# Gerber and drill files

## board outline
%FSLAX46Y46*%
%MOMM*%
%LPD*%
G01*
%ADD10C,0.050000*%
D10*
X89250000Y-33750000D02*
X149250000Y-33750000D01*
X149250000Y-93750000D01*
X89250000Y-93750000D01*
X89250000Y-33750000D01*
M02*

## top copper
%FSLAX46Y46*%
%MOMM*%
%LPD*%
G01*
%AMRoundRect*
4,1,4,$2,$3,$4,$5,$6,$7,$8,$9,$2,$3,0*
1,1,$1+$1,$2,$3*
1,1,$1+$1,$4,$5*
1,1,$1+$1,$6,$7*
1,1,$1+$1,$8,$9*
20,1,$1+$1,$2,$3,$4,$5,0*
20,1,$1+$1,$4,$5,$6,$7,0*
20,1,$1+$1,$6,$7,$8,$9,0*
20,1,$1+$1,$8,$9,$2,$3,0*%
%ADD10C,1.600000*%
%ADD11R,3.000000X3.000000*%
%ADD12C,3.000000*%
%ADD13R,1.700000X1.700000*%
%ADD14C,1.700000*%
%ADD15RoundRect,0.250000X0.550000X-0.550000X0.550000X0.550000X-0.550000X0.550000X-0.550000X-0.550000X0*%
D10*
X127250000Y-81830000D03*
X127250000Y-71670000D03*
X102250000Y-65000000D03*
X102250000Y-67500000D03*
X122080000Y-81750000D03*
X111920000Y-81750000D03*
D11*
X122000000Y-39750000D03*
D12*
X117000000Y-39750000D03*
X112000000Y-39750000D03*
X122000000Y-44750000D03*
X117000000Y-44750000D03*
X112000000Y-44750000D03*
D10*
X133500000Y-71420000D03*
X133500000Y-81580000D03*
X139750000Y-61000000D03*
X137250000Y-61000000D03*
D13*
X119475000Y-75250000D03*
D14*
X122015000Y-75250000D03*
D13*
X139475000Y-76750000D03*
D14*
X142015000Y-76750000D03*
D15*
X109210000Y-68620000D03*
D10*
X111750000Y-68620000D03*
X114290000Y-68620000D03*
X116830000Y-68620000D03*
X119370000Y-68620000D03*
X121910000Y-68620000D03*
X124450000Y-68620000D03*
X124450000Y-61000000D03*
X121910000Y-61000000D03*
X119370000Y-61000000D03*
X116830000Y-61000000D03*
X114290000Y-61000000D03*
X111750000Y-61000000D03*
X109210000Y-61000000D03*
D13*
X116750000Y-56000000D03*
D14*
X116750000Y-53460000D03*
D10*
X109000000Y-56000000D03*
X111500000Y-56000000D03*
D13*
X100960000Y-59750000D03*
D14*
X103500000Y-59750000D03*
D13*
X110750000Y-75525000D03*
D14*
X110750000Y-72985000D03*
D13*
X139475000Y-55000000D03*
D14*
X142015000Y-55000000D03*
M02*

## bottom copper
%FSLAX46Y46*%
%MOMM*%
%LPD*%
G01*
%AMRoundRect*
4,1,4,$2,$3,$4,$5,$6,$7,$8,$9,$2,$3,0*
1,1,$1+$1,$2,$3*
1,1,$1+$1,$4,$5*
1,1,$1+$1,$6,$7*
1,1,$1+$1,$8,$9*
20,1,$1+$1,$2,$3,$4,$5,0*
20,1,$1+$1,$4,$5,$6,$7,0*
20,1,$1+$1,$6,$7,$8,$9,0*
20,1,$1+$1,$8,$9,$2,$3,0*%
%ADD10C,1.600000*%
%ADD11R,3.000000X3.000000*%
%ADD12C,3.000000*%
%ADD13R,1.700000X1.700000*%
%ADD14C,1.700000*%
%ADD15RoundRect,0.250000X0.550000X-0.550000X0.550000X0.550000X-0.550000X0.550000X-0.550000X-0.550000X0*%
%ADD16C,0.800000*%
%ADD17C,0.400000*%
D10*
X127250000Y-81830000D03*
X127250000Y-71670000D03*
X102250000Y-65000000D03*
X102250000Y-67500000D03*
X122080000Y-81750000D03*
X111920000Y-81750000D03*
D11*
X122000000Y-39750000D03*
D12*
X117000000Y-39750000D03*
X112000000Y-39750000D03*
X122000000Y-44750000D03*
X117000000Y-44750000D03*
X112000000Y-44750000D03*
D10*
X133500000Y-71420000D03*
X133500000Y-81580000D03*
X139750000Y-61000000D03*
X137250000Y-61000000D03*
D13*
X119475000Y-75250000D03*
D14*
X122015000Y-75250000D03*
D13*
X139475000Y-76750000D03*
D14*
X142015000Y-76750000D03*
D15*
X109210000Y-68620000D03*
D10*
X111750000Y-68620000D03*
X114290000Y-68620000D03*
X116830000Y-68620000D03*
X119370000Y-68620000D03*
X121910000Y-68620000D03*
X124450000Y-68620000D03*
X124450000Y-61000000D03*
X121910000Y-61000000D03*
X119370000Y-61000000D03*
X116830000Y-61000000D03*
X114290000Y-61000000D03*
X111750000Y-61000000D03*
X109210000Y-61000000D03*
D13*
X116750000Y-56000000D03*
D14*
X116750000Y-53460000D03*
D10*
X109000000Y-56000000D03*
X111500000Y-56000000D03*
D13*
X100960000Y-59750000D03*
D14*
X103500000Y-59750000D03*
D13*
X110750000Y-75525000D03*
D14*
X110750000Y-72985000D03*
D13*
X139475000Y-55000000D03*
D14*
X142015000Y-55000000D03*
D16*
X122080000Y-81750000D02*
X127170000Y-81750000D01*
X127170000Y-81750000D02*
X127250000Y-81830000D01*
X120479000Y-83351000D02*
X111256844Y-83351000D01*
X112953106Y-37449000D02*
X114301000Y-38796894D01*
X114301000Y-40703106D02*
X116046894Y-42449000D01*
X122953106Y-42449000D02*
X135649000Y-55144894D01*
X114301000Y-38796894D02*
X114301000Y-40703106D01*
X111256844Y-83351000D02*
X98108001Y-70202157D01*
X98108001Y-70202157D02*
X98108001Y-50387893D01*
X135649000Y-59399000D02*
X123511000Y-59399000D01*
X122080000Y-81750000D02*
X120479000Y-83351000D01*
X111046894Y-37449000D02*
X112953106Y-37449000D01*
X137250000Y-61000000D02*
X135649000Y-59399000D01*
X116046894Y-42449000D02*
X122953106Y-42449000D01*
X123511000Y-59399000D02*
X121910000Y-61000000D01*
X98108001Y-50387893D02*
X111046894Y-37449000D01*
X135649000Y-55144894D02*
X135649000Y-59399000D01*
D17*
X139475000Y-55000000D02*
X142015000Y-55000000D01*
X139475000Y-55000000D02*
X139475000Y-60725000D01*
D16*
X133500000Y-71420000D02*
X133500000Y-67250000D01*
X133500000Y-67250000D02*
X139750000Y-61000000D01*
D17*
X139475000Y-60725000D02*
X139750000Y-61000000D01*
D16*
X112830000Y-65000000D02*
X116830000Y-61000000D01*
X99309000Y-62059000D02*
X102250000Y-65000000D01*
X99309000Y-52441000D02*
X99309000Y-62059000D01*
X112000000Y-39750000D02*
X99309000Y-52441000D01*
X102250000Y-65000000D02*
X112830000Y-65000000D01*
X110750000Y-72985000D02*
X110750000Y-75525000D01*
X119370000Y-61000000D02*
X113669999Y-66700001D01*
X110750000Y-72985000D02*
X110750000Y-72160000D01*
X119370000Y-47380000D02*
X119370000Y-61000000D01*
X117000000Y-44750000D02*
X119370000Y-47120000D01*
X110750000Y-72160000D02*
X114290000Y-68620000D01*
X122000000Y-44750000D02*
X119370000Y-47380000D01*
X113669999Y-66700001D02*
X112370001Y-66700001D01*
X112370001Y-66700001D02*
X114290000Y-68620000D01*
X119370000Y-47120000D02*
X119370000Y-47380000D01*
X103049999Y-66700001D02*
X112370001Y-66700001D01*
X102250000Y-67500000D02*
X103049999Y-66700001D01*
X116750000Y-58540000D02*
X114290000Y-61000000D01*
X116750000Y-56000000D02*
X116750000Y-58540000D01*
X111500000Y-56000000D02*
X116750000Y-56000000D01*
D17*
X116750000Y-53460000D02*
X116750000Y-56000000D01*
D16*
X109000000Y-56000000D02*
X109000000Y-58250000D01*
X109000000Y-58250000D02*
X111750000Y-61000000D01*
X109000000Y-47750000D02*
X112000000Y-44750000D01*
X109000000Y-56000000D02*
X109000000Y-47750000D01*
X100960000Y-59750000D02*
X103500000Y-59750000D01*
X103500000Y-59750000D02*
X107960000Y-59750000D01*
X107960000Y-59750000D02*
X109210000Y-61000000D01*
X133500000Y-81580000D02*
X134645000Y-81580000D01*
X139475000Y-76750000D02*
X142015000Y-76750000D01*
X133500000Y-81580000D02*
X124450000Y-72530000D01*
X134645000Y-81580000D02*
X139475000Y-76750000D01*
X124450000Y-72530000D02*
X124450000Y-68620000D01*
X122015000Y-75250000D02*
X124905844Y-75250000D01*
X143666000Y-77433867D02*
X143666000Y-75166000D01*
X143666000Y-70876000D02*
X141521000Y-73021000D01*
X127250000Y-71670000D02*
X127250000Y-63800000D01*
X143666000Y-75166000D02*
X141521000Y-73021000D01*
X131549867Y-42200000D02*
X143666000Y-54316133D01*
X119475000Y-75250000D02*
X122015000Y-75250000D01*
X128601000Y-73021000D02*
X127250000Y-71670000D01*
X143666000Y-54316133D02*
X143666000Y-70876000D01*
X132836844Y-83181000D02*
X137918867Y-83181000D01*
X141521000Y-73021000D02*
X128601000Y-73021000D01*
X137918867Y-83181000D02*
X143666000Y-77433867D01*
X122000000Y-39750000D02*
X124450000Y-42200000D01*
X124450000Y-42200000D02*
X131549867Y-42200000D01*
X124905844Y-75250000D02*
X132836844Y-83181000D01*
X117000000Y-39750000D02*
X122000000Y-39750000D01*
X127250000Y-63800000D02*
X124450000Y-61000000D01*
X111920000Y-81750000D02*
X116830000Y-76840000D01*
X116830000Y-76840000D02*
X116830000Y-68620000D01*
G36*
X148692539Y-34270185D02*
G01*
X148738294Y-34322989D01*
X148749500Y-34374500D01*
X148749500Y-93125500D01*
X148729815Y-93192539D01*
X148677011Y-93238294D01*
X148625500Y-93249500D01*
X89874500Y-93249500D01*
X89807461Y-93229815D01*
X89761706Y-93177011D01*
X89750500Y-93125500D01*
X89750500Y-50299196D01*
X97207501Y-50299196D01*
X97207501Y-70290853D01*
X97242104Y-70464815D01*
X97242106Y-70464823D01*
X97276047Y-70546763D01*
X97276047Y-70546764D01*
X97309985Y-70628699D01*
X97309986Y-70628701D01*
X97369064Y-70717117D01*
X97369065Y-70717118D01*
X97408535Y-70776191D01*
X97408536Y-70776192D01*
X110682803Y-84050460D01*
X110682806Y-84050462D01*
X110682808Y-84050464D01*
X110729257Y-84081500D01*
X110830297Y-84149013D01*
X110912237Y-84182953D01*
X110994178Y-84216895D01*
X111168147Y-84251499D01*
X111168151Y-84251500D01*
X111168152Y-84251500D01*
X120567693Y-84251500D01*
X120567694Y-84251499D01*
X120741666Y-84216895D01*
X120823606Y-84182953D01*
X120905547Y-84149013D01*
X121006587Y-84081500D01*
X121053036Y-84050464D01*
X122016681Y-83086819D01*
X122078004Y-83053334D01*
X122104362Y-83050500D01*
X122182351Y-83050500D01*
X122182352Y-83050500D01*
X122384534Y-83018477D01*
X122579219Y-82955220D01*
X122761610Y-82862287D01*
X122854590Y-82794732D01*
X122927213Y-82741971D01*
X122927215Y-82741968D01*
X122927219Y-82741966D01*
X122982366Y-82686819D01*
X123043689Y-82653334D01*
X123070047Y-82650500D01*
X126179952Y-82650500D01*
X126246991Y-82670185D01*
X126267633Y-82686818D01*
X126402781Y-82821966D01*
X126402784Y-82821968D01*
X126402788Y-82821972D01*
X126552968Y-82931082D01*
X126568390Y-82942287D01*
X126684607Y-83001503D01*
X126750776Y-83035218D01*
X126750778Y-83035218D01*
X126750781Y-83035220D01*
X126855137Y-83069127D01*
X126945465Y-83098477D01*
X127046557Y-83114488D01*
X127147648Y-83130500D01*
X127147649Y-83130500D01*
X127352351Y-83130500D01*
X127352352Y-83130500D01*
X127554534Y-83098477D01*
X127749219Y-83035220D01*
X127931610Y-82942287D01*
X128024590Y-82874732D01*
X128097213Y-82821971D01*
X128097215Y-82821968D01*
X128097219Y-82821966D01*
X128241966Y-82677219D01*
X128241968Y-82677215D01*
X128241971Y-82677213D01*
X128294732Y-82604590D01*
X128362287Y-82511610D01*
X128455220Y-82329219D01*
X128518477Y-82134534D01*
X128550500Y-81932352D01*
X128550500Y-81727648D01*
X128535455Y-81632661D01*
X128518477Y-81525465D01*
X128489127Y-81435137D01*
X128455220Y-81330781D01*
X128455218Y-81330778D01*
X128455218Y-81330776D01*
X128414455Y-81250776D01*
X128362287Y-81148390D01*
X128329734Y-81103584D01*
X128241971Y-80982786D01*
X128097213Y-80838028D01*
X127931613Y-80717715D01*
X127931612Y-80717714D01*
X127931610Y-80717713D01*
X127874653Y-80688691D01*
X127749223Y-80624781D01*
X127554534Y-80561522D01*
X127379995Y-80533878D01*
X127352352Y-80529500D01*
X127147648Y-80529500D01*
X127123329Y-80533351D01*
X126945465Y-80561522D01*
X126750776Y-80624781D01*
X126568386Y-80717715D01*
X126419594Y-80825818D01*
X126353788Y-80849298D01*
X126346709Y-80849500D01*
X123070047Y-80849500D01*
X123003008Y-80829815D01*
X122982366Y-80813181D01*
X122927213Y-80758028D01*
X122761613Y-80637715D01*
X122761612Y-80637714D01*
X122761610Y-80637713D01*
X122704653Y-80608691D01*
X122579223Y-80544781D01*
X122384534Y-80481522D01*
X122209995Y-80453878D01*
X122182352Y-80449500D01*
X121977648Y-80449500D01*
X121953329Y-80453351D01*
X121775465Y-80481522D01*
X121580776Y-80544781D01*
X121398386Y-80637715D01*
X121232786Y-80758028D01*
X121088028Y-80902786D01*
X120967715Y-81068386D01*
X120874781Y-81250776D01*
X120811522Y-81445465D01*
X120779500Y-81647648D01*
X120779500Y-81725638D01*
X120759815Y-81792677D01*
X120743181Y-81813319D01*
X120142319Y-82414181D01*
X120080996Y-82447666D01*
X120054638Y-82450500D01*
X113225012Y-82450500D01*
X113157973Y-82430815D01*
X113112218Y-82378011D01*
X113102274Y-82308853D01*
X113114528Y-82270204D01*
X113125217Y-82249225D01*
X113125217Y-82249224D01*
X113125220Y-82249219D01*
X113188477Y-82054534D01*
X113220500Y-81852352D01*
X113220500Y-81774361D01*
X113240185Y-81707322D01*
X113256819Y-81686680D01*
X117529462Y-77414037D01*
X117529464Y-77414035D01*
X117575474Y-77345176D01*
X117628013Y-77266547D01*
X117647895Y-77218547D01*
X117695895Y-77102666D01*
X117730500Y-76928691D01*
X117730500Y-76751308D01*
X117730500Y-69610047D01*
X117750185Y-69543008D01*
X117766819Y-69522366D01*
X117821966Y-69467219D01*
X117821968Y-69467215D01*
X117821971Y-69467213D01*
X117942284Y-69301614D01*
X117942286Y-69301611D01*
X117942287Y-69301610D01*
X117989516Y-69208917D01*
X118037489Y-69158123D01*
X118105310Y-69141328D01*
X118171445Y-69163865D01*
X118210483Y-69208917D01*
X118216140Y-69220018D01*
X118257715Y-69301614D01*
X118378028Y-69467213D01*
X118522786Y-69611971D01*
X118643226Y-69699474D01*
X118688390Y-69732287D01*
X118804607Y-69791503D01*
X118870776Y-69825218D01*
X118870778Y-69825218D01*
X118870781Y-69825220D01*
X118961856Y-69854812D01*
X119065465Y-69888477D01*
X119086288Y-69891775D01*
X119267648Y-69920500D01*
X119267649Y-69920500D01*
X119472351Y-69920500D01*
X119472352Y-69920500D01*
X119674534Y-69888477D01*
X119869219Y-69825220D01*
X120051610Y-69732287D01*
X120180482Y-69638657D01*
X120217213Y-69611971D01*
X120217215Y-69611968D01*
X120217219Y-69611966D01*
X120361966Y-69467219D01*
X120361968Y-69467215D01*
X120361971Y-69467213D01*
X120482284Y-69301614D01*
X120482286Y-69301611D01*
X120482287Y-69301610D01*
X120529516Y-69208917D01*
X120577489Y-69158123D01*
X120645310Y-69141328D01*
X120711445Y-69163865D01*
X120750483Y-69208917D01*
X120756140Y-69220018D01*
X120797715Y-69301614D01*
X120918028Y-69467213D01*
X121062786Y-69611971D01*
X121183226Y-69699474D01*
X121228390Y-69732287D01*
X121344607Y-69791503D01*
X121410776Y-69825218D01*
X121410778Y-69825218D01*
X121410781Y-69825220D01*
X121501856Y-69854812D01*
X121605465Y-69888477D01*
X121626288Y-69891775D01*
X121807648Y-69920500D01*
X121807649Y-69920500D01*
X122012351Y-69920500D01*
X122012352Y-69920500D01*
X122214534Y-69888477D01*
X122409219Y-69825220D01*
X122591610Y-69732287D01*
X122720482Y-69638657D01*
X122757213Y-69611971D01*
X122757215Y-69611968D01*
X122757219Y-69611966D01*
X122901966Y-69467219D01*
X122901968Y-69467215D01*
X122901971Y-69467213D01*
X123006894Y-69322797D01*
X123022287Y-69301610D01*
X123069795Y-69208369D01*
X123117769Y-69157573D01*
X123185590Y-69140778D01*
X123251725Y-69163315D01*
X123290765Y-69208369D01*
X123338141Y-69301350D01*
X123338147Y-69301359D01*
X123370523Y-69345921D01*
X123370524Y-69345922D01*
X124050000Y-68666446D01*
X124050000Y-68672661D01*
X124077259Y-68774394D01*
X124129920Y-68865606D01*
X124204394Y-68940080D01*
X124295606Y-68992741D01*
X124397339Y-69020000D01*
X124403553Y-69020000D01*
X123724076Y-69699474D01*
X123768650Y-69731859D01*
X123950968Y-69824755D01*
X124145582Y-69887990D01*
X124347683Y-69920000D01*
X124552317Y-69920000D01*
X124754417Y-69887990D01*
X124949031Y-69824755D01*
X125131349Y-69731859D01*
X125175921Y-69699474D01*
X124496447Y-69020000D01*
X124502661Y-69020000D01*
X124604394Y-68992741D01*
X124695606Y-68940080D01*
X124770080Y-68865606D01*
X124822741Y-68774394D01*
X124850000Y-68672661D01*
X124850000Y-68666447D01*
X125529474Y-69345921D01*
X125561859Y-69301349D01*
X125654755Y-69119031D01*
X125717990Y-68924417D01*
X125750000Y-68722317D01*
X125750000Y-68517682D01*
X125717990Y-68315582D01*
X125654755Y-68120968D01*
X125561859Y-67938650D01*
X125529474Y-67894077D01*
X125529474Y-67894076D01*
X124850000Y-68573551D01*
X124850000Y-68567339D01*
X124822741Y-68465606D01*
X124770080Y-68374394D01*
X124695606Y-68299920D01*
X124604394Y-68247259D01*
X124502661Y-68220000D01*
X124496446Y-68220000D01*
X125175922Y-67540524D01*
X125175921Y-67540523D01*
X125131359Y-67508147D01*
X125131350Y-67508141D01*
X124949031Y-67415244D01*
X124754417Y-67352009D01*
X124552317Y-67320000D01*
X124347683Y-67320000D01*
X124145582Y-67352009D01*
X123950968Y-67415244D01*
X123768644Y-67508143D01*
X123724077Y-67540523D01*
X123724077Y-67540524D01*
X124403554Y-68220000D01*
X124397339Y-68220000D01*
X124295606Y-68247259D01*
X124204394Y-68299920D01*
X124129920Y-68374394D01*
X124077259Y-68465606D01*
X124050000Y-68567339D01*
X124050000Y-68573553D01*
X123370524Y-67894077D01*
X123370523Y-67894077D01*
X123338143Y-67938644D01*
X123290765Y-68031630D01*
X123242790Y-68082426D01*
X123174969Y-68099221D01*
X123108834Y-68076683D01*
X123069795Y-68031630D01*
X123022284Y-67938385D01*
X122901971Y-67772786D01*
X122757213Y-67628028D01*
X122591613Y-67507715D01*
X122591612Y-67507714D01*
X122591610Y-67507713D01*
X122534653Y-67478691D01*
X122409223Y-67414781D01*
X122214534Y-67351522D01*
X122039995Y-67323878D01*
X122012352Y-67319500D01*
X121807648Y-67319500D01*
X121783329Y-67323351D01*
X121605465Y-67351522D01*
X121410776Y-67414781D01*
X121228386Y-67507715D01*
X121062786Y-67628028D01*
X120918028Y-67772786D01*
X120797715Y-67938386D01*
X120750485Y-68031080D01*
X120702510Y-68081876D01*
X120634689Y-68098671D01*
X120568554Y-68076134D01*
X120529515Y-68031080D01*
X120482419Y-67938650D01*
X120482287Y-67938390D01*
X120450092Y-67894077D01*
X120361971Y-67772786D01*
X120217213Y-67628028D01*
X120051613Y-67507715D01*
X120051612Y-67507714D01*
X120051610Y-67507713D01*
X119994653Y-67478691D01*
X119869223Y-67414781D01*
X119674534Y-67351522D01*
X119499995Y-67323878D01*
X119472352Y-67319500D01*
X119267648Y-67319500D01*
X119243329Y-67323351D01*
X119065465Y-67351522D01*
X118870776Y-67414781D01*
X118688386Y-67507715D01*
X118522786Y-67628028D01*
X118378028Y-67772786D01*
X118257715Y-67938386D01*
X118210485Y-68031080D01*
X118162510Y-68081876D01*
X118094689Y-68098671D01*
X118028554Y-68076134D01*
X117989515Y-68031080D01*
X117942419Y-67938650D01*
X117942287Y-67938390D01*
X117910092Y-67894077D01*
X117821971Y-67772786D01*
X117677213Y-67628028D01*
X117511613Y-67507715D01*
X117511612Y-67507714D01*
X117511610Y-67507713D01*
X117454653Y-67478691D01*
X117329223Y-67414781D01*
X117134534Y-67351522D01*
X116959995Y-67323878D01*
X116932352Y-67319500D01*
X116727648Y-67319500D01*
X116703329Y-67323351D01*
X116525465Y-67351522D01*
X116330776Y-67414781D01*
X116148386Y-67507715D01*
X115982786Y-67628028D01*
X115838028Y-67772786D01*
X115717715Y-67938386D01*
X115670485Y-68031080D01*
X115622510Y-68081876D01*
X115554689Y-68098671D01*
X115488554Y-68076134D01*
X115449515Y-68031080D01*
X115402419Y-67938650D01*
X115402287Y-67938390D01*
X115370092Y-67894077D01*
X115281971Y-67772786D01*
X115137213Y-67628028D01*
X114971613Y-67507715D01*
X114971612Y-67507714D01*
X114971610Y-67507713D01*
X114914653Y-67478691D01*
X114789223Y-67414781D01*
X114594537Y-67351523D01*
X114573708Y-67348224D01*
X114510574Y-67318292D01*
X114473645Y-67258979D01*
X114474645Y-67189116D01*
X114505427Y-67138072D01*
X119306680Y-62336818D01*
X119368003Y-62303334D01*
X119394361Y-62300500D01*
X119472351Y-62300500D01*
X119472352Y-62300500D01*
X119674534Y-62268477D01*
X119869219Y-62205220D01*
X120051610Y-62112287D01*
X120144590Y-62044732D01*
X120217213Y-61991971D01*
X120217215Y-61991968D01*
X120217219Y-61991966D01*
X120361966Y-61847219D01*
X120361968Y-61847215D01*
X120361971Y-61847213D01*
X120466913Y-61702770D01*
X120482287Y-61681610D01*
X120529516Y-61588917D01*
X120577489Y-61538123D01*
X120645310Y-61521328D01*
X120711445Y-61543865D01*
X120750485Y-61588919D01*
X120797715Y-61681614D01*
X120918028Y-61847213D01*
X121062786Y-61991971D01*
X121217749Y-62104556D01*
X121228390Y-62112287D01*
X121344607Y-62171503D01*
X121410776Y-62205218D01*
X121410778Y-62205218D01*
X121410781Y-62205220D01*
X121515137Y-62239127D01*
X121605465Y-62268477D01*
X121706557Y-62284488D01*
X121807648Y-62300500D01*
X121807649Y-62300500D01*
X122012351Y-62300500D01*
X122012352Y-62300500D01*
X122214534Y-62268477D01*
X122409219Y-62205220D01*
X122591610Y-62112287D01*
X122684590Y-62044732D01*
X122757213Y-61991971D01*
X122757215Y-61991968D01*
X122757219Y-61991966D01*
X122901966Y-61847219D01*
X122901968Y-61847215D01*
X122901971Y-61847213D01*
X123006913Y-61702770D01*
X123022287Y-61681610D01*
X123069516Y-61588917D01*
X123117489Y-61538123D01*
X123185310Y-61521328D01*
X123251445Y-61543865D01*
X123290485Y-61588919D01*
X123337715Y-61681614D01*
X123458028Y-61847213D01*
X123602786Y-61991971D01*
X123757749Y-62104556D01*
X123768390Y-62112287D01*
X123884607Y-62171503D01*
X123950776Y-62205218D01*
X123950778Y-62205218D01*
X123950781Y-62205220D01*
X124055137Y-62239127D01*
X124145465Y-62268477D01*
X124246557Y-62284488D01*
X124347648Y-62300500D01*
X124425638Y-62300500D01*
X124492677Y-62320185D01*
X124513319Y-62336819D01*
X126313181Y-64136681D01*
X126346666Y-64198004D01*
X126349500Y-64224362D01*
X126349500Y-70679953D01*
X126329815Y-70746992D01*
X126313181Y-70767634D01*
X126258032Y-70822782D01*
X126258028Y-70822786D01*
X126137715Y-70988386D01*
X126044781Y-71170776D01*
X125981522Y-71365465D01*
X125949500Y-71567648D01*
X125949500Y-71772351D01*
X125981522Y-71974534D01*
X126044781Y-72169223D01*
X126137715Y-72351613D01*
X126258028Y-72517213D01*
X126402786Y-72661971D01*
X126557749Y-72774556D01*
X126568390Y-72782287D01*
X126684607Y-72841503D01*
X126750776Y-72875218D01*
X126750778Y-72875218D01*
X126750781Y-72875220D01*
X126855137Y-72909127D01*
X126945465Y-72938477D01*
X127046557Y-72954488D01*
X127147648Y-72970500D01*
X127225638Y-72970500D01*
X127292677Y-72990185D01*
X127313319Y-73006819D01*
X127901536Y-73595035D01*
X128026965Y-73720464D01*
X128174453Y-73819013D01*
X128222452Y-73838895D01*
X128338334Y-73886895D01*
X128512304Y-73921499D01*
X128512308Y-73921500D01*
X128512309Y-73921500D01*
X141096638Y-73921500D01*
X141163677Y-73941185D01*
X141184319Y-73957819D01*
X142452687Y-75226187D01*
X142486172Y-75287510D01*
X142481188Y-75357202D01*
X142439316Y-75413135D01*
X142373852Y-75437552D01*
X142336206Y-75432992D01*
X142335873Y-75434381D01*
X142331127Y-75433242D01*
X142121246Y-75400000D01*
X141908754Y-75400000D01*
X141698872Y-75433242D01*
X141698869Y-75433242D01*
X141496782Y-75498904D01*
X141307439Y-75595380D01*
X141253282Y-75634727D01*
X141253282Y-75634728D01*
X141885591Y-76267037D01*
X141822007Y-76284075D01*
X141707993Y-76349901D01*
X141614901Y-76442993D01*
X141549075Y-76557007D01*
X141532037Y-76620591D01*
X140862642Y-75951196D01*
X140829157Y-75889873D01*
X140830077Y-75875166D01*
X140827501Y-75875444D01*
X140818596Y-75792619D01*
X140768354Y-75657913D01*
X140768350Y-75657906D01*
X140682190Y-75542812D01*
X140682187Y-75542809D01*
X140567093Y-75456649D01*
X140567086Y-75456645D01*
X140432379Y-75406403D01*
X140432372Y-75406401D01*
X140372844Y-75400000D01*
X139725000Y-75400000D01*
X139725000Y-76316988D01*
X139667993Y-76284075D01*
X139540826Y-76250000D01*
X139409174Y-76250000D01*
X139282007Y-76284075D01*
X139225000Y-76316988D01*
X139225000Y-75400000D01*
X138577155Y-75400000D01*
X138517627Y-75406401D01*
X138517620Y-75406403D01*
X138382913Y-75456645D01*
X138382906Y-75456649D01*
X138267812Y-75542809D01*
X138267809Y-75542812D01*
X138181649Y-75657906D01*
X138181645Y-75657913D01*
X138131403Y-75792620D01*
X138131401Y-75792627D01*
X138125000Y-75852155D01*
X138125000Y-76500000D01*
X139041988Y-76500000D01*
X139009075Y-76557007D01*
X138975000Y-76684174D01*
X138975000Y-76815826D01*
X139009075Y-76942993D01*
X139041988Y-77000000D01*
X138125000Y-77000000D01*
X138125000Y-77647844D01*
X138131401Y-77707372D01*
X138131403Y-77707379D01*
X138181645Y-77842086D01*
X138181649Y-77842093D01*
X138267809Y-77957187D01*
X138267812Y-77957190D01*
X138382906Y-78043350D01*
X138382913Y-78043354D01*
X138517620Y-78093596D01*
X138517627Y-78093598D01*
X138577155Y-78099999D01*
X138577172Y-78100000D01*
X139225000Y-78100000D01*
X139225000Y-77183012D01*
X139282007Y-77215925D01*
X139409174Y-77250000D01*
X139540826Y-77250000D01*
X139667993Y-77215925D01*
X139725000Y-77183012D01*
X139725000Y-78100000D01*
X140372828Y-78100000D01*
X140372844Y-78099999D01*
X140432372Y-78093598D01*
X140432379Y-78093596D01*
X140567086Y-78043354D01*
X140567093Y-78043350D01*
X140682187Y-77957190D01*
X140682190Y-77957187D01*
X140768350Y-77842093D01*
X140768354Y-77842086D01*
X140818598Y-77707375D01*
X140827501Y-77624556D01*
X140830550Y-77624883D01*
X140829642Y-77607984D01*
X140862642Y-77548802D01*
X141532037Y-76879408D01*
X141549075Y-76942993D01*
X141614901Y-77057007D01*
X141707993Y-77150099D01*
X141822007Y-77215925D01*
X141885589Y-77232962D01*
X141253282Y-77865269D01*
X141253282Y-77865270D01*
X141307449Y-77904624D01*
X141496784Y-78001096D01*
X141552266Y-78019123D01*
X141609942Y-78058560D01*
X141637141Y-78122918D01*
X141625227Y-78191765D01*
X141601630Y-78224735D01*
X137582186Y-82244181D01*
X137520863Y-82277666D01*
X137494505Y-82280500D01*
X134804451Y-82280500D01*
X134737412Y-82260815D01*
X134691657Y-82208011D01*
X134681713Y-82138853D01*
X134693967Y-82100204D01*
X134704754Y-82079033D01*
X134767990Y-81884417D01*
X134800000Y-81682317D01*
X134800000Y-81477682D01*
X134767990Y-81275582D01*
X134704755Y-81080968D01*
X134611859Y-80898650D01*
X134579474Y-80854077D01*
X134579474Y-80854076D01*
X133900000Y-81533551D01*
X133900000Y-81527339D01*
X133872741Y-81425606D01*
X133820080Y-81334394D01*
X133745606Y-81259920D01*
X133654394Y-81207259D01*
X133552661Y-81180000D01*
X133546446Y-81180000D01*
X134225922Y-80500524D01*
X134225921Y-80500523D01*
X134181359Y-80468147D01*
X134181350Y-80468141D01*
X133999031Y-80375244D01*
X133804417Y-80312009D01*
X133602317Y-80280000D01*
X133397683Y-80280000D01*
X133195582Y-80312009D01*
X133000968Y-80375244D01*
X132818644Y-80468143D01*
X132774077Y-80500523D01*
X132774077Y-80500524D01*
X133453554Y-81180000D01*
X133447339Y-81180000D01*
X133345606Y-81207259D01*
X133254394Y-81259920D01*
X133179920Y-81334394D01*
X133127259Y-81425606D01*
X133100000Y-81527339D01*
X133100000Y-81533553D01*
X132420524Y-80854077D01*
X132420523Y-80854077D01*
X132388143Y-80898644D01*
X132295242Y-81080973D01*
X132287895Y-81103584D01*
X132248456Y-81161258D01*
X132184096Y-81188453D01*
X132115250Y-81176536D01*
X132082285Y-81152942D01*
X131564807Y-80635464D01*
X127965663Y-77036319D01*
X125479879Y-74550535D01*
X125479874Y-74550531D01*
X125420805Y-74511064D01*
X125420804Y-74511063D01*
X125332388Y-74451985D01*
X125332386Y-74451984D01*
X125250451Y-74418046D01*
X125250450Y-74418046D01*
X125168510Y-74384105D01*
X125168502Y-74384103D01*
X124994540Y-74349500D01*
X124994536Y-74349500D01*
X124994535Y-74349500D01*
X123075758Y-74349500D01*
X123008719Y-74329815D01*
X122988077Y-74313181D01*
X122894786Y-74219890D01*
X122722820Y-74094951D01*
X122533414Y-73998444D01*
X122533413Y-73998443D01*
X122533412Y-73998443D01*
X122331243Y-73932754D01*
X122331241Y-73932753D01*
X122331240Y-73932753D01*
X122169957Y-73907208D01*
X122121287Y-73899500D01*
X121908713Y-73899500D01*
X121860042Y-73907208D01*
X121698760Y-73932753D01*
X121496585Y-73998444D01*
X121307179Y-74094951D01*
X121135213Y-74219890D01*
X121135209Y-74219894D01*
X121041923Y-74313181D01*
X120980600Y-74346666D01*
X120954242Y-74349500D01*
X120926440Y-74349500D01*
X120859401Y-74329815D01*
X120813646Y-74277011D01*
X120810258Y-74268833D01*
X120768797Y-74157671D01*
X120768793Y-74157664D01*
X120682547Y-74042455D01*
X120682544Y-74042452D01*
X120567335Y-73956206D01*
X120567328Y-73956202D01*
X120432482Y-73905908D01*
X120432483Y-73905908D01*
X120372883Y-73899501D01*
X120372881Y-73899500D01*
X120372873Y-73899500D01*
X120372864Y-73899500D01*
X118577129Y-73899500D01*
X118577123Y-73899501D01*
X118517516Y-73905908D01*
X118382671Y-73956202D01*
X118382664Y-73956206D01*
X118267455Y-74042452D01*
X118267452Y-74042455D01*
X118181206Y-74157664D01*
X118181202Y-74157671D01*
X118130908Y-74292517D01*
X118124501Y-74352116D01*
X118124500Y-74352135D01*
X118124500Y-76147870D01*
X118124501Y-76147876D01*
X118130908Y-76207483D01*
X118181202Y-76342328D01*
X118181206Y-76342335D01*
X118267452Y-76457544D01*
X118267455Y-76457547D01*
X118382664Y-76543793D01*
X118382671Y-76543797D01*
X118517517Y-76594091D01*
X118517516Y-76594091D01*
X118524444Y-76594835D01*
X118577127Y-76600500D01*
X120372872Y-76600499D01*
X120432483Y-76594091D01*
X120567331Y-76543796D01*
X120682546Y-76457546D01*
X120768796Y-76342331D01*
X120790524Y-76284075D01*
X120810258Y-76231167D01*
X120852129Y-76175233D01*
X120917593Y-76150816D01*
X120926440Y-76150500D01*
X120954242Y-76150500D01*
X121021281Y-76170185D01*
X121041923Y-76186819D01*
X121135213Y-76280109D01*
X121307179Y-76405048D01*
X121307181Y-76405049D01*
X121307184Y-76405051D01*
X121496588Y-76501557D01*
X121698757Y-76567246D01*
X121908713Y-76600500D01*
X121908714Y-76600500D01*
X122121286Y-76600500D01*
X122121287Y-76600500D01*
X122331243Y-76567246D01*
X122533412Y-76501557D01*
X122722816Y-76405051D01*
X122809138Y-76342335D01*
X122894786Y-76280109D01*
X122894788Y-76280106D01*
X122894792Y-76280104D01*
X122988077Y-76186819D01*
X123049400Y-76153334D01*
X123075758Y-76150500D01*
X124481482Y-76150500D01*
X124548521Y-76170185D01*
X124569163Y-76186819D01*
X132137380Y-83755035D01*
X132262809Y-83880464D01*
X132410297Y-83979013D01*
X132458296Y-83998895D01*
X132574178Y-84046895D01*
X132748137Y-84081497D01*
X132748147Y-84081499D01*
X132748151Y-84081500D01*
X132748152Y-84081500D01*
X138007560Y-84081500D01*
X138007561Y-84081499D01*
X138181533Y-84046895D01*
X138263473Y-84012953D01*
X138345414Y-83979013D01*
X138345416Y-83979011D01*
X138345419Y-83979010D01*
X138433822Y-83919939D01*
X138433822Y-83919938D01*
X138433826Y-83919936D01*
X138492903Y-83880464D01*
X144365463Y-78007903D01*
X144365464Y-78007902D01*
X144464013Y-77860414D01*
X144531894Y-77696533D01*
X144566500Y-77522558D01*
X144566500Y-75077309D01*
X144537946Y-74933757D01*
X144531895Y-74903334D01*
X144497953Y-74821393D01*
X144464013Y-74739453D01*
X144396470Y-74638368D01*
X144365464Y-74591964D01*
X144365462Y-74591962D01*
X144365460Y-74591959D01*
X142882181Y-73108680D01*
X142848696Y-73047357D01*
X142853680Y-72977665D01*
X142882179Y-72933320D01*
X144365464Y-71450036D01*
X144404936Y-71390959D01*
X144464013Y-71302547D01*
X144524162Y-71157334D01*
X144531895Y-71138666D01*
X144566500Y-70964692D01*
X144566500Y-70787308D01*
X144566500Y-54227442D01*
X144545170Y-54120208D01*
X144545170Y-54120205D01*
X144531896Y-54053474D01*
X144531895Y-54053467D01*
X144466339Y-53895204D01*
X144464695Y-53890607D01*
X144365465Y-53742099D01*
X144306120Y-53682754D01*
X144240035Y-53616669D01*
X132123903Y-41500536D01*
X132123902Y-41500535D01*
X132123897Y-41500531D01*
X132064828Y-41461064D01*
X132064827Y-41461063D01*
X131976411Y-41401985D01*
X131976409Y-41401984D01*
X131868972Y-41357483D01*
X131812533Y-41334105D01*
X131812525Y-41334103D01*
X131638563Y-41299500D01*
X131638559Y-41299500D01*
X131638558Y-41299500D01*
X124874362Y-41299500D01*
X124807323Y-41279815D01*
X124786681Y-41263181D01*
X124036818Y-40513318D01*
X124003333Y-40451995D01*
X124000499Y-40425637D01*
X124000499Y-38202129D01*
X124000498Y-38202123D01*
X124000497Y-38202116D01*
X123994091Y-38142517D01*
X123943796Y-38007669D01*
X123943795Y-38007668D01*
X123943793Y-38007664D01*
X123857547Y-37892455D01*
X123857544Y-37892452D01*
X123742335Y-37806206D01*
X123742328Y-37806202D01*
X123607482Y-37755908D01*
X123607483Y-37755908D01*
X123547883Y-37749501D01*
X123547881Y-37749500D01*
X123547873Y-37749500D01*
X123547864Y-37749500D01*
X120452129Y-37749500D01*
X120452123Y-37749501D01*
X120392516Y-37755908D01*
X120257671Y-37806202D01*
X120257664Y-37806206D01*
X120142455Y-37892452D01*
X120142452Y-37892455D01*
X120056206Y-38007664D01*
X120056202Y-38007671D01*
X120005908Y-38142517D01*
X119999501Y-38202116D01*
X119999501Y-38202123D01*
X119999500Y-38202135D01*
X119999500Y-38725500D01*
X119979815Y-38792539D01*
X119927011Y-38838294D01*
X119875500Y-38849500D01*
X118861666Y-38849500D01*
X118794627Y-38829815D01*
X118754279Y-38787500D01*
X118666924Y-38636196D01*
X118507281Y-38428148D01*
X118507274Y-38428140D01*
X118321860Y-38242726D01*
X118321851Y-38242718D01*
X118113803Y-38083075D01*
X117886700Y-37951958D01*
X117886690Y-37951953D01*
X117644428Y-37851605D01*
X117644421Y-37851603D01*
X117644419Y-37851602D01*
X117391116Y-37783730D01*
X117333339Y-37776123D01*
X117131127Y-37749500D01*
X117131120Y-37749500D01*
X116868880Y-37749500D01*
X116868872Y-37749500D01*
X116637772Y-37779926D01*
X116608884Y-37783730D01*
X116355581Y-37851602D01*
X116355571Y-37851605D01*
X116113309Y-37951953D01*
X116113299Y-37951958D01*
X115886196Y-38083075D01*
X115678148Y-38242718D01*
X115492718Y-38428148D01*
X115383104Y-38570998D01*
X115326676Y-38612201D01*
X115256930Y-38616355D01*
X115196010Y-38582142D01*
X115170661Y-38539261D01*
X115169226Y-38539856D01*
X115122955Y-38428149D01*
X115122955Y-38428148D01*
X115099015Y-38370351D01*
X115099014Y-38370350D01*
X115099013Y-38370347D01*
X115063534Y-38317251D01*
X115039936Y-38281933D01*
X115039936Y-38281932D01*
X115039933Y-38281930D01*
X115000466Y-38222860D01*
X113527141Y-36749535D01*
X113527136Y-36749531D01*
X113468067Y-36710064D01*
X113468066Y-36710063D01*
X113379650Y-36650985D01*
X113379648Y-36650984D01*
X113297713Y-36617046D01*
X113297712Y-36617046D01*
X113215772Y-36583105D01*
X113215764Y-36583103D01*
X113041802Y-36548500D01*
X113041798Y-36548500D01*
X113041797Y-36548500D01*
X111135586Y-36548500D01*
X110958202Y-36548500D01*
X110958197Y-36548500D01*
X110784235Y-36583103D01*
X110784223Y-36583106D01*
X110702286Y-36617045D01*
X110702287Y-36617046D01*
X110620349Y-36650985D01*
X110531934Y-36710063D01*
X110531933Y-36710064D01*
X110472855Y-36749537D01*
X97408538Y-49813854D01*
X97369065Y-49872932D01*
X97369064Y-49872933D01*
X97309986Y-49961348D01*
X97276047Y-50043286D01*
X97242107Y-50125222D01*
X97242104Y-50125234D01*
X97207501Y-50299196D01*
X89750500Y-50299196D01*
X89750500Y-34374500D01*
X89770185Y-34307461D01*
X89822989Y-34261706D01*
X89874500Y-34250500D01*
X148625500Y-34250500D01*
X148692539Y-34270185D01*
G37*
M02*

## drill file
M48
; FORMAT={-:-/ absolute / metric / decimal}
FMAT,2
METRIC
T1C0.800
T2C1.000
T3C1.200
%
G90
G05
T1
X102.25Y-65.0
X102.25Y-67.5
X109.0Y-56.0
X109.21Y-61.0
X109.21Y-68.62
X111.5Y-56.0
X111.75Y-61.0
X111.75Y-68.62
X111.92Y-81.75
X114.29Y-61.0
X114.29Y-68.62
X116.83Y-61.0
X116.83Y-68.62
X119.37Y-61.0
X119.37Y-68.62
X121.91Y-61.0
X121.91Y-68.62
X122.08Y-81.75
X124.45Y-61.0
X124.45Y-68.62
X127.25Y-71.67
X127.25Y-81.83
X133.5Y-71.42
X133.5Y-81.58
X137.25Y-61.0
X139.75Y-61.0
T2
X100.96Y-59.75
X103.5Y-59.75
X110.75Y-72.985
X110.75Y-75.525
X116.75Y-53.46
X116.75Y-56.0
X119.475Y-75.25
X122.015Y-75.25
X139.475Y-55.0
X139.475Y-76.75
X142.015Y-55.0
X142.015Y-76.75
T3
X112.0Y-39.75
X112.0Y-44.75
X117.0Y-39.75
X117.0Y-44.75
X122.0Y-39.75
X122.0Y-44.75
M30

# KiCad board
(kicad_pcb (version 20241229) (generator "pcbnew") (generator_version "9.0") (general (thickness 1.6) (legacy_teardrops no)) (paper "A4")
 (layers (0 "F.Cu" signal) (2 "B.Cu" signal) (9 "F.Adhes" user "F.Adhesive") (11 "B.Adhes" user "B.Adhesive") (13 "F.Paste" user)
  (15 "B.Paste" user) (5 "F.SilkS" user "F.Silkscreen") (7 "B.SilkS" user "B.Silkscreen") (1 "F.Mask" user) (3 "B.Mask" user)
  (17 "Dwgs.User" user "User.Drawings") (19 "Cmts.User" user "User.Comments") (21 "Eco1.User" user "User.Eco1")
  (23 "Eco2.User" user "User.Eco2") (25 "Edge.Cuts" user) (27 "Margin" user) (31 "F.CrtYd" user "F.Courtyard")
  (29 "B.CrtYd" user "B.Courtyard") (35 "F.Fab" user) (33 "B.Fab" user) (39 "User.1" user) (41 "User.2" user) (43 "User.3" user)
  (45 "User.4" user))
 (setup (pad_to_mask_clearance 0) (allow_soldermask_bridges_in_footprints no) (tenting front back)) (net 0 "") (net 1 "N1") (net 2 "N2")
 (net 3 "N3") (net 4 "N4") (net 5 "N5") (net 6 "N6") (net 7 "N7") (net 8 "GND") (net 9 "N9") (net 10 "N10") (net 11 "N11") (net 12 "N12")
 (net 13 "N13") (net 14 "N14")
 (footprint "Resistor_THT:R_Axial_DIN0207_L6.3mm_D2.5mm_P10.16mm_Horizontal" (layer "F.Cu") (at 127.25 81.83 90)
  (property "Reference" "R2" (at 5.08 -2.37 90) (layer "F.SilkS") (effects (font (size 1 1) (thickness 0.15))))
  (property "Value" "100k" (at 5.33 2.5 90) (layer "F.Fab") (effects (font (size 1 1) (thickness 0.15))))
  (pad "1" thru_hole circle (at 0 0 90) (size 1.6 1.6) (drill 0.8) (layers "*.Cu" "*.Mask") (remove_unused_layers no) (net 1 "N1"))
  (pad "2" thru_hole circle (at 10.16 0 90) (size 1.6 1.6) (drill 0.8) (layers "*.Cu" "*.Mask") (remove_unused_layers no) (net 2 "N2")))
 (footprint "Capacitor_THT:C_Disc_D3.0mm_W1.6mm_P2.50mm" (layer "F.Cu") (at 102.25 65 -90)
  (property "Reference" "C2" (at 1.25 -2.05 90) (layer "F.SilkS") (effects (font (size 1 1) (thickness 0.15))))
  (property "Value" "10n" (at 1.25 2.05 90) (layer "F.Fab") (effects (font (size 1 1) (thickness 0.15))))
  (pad "1" thru_hole circle (at 0 0 270) (size 1.6 1.6) (drill 0.8) (layers "*.Cu" "*.Mask") (remove_unused_layers no) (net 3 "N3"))
  (pad "2" thru_hole circle (at 2.5 0 270) (size 1.6 1.6) (drill 0.8) (layers "*.Cu" "*.Mask") (remove_unused_layers no) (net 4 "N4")))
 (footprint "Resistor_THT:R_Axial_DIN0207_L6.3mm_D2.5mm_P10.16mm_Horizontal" (layer "F.Cu") (at 122.08 81.75 180)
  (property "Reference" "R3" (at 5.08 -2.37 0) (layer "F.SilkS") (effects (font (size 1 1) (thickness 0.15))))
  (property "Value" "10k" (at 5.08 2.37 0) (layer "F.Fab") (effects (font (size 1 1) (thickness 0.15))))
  (pad "1" thru_hole circle (at 0 0 180) (size 1.6 1.6) (drill 0.8) (layers "*.Cu" "*.Mask") (remove_unused_layers no) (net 1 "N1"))
  (pad "2" thru_hole circle (at 10.16 0 180) (size 1.6 1.6) (drill 0.8) (layers "*.Cu" "*.Mask") (remove_unused_layers no) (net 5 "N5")))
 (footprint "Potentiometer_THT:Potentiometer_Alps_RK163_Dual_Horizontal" (layer "F.Cu") (at 122 39.75 -90)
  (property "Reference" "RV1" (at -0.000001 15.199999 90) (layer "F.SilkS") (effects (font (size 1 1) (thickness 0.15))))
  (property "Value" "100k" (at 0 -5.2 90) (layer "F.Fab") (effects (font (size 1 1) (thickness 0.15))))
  (pad "1" thru_hole rect (at 0 0 90) (size 3 3) (drill 1.2) (layers "*.Cu" "*.Mask") (remove_unused_layers no) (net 2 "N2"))
  (pad "2" thru_hole circle (at 0 5 90) (size 3 3) (drill 1.2) (layers "*.Cu" "*.Mask") (remove_unused_layers no) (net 2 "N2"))
  (pad "3" thru_hole circle (at 0 10 90) (size 3 3) (drill 1.2) (layers "*.Cu" "*.Mask") (remove_unused_layers no) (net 3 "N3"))
  (pad "4" thru_hole circle (at 5 0 90) (size 3 3) (drill 1.2) (layers "*.Cu" "*.Mask") (remove_unused_layers no) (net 4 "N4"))
  (pad "5" thru_hole circle (at 5 5 90) (size 3 3) (drill 1.2) (layers "*.Cu" "*.Mask") (remove_unused_layers no) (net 4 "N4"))
  (pad "6" thru_hole circle (at 5 10 90) (size 3 3) (drill 1.2) (layers "*.Cu" "*.Mask") (remove_unused_layers no) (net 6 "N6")))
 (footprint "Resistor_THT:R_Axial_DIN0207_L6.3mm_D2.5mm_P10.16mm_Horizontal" (layer "F.Cu") (at 133.5 71.42 -90)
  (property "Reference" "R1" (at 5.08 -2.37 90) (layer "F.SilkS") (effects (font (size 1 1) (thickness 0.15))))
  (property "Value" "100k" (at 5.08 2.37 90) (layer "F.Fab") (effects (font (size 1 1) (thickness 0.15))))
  (pad "1" thru_hole circle (at 0 0 270) (size 1.6 1.6) (drill 0.8) (layers "*.Cu" "*.Mask") (remove_unused_layers no) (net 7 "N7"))
  (pad "2" thru_hole circle (at 10.16 0 270) (size 1.6 1.6) (drill 0.8) (layers "*.Cu" "*.Mask") (remove_unused_layers no) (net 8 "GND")))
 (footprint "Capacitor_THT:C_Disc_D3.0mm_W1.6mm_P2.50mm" (layer "F.Cu") (at 139.75 61 180)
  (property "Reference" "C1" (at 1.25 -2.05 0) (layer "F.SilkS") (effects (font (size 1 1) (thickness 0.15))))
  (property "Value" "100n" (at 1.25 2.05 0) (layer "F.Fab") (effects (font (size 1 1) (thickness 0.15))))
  (pad "1" thru_hole circle (at 0 0 180) (size 1.6 1.6) (drill 0.8) (layers "*.Cu" "*.Mask") (remove_unused_layers no) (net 7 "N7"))
  (pad "2" thru_hole circle (at 2.5 0 180) (size 1.6 1.6) (drill 0.8) (layers "*.Cu" "*.Mask") (remove_unused_layers no) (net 1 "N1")))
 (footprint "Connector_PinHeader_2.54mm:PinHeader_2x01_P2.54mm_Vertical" (layer "F.Cu") (at 119.475 75.25)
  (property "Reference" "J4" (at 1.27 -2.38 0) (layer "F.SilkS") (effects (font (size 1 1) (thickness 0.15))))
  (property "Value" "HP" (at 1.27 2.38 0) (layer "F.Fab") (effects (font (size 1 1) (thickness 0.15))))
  (pad "1" thru_hole rect (at 0 0) (size 1.7 1.7) (drill 1) (layers "*.Cu" "*.Mask") (remove_unused_layers no) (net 2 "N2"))
  (pad "2" thru_hole circle (at 2.54 0) (size 1.7 1.7) (drill 1) (layers "*.Cu" "*.Mask") (remove_unused_layers no) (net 2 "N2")))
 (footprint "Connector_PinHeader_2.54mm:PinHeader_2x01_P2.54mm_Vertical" (layer "F.Cu") (at 139.475 76.75)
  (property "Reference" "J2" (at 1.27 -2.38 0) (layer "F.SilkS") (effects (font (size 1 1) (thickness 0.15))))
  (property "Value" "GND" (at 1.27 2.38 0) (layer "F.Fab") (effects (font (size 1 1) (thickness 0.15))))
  (pad "1" thru_hole rect (at 0 0) (size 1.7 1.7) (drill 1) (layers "*.Cu" "*.Mask") (remove_unused_layers no) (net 8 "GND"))
  (pad "2" thru_hole circle (at 2.54 0) (size 1.7 1.7) (drill 1) (layers "*.Cu" "*.Mask") (remove_unused_layers no) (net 8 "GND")))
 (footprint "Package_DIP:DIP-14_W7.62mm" (layer "F.Cu") (at 109.21 68.62 90)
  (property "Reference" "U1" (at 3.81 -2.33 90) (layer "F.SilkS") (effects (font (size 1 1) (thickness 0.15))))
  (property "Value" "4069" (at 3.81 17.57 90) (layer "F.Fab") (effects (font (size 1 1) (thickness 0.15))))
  (pad "1" thru_hole roundrect (at 0 0 90) (size 1.6 1.6) (drill 0.8) (layers "*.Cu" "*.Mask") (remove_unused_layers no)
   (roundrect_rratio 0.15625) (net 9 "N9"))
  (pad "2" thru_hole circle (at 0 2.54 90) (size 1.6 1.6) (drill 0.8) (layers "*.Cu" "*.Mask") (remove_unused_layers no) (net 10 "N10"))
  (pad "3" thru_hole circle (at 0 5.08 90) (size 1.6 1.6) (drill 0.8) (layers "*.Cu" "*.Mask") (remove_unused_layers no) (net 4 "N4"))
  (pad "4" thru_hole circle (at 0 7.62 90) (size 1.6 1.6) (drill 0.8) (layers "*.Cu" "*.Mask") (remove_unused_layers no) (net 5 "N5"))
  (pad "5" thru_hole circle (at 0 10.16 90) (size 1.6 1.6) (drill 0.8) (layers "*.Cu" "*.Mask") (remove_unused_layers no) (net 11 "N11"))
  (pad "6" thru_hole circle (at 0 12.7 90) (size 1.6 1.6) (drill 0.8) (layers "*.Cu" "*.Mask") (remove_unused_layers no) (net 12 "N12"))
  (pad "7" thru_hole circle (at 0 15.24 90) (size 1.6 1.6) (drill 0.8) (layers "*.Cu" "*.Mask") (remove_unused_layers no) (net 8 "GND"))
  (pad "8" thru_hole circle (at 7.62 15.24 90) (size 1.6 1.6) (drill 0.8) (layers "*.Cu" "*.Mask") (remove_unused_layers no) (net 2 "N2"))
  (pad "9" thru_hole circle (at 7.62 12.7 90) (size 1.6 1.6) (drill 0.8) (layers "*.Cu" "*.Mask") (remove_unused_layers no) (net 1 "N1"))
  (pad "10" thru_hole circle (at 7.62 10.16 90) (size 1.6 1.6) (drill 0.8) (layers "*.Cu" "*.Mask") (remove_unused_layers no) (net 4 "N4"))
  (pad "11" thru_hole circle (at 7.62 7.62 90) (size 1.6 1.6) (drill 0.8) (layers "*.Cu" "*.Mask") (remove_unused_layers no) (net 3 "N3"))
  (pad "12" thru_hole circle (at 7.62 5.08 90) (size 1.6 1.6) (drill 0.8) (layers "*.Cu" "*.Mask") (remove_unused_layers no) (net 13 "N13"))
  (pad "13" thru_hole circle (at 7.62 2.54 90) (size 1.6 1.6) (drill 0.8) (layers "*.Cu" "*.Mask") (remove_unused_layers no) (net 6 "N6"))
  (pad "14" thru_hole circle (at 7.62 0 90) (size 1.6 1.6) (drill 0.8) (layers "*.Cu" "*.Mask") (remove_unused_layers no) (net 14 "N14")))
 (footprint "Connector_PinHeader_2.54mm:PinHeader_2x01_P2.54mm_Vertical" (layer "F.Cu") (at 116.75 56 90)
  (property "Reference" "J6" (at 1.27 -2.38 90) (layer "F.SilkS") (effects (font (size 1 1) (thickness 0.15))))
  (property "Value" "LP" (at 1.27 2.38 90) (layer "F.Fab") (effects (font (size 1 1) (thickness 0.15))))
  (pad "1" thru_hole rect (at 0 0 90) (size 1.7 1.7) (drill 1) (layers "*.Cu" "*.Mask") (remove_unused_layers no) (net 13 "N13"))
  (pad "2" thru_hole circle (at 2.54 0 90) (size 1.7 1.7) (drill 1) (layers "*.Cu" "*.Mask") (remove_unused_layers no) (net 13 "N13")))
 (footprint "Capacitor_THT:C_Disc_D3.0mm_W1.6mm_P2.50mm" (layer "F.Cu") (at 109 56)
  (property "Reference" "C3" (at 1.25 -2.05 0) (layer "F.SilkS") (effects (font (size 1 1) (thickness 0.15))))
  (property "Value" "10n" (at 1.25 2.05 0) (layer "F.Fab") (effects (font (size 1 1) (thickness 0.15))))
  (pad "1" thru_hole circle (at 0 0) (size 1.6 1.6) (drill 0.8) (layers "*.Cu" "*.Mask") (remove_unused_layers no) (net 6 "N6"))
  (pad "2" thru_hole circle (at 2.5 0) (size 1.6 1.6) (drill 0.8) (layers "*.Cu" "*.Mask") (remove_unused_layers no) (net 13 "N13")))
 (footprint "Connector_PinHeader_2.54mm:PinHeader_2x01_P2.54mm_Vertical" (layer "F.Cu") (at 100.96 59.75)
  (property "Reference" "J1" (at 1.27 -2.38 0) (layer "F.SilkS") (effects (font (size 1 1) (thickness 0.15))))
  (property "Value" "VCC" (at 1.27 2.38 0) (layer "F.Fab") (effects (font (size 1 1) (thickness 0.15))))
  (pad "1" thru_hole rect (at 0 0) (size 1.7 1.7) (drill 1) (layers "*.Cu" "*.Mask") (remove_unused_layers no) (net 14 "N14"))
  (pad "2" thru_hole circle (at 2.54 0) (size 1.7 1.7) (drill 1) (layers "*.Cu" "*.Mask") (remove_unused_layers no) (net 14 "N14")))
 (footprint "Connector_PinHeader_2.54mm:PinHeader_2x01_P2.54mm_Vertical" (layer "F.Cu") (at 110.75 75.525 90)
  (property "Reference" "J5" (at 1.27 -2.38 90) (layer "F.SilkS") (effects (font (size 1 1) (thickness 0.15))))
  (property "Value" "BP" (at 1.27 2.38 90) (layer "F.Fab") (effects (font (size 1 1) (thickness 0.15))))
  (pad "1" thru_hole rect (at 0 0 90) (size 1.7 1.7) (drill 1) (layers "*.Cu" "*.Mask") (remove_unused_layers no) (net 4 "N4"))
  (pad "2" thru_hole circle (at 2.54 0 90) (size 1.7 1.7) (drill 1) (layers "*.Cu" "*.Mask") (remove_unused_layers no) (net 4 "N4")))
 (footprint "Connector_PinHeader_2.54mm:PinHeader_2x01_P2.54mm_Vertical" (layer "F.Cu") (at 139.475 55)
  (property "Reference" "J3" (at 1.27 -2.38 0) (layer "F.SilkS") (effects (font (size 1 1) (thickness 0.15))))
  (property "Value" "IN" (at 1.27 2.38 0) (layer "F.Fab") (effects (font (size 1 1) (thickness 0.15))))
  (pad "1" thru_hole rect (at 0 0) (size 1.7 1.7) (drill 1) (layers "*.Cu" "*.Mask") (remove_unused_layers no) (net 7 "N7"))
  (pad "2" thru_hole circle (at 2.54 0) (size 1.7 1.7) (drill 1) (layers "*.Cu" "*.Mask") (remove_unused_layers no) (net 7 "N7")))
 (gr_rect (start 89.25 33.75) (end 149.25 93.75) (stroke (width 0.05) (type default)) (fill no) (layer "Edge.Cuts"))
 (segment (start 122.08 81.75) (end 127.17 81.75) (width 0.8) (layer "B.Cu") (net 1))
 (segment (start 127.17 81.75) (end 127.25 81.83) (width 0.8) (layer "B.Cu") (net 1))
 (segment (start 120.479 83.351) (end 111.256844 83.351) (width 0.8) (layer "B.Cu") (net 1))
 (segment (start 112.953106 37.449) (end 114.301 38.796894) (width 0.8) (layer "B.Cu") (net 1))
 (segment (start 114.301 40.703106) (end 116.046894 42.449) (width 0.8) (layer "B.Cu") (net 1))
 (segment (start 122.953106 42.449) (end 135.649 55.144894) (width 0.8) (layer "B.Cu") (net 1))
 (segment (start 114.301 38.796894) (end 114.301 40.703106) (width 0.8) (layer "B.Cu") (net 1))
 (segment (start 111.256844 83.351) (end 98.108001 70.202157) (width 0.8) (layer "B.Cu") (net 1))
 (segment (start 98.108001 70.202157) (end 98.108001 50.387893) (width 0.8) (layer "B.Cu") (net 1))
 (segment (start 135.649 59.399) (end 123.511 59.399) (width 0.8) (layer "B.Cu") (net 1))
 (segment (start 122.08 81.75) (end 120.479 83.351) (width 0.8) (layer "B.Cu") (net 1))
 (segment (start 111.046894 37.449) (end 112.953106 37.449) (width 0.8) (layer "B.Cu") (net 1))
 (segment (start 137.25 61) (end 135.649 59.399) (width 0.8) (layer "B.Cu") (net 1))
 (segment (start 116.046894 42.449) (end 122.953106 42.449) (width 0.8) (layer "B.Cu") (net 1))
 (segment (start 123.511 59.399) (end 121.91 61) (width 0.8) (layer "B.Cu") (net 1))
 (segment (start 98.108001 50.387893) (end 111.046894 37.449) (width 0.8) (layer "B.Cu") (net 1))
 (segment (start 135.649 55.144894) (end 135.649 59.399) (width 0.8) (layer "B.Cu") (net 1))
 (segment (start 139.475 55) (end 142.015 55) (width 0.4) (layer "B.Cu") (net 7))
 (segment (start 139.475 55) (end 139.475 60.725) (width 0.4) (layer "B.Cu") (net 7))
 (segment (start 133.5 71.42) (end 133.5 67.25) (width 0.8) (layer "B.Cu") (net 7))
 (segment (start 133.5 67.25) (end 139.75 61) (width 0.8) (layer "B.Cu") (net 7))
 (segment (start 139.475 60.725) (end 139.75 61) (width 0.4) (layer "B.Cu") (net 7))
 (segment (start 112.83 65) (end 116.83 61) (width 0.8) (layer "B.Cu") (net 3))
 (segment (start 99.309 62.059) (end 102.25 65) (width 0.8) (layer "B.Cu") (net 3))
 (segment (start 99.309 52.441) (end 99.309 62.059) (width 0.8) (layer "B.Cu") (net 3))
 (segment (start 112 39.75) (end 99.309 52.441) (width 0.8) (layer "B.Cu") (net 3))
 (segment (start 102.25 65) (end 112.83 65) (width 0.8) (layer "B.Cu") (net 3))
 (segment (start 110.75 72.985) (end 110.75 75.525) (width 0.8) (layer "B.Cu") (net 4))
 (segment (start 119.37 61) (end 113.669999 66.700001) (width 0.8) (layer "B.Cu") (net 4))
 (segment (start 110.75 72.985) (end 110.75 72.16) (width 0.8) (layer "B.Cu") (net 4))
 (segment (start 119.37 47.38) (end 119.37 61) (width 0.8) (layer "B.Cu") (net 4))
 (segment (start 117 44.75) (end 119.37 47.12) (width 0.8) (layer "B.Cu") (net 4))
 (segment (start 110.75 72.16) (end 114.29 68.62) (width 0.8) (layer "B.Cu") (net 4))
 (segment (start 122 44.75) (end 119.37 47.38) (width 0.8) (layer "B.Cu") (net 4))
 (segment (start 113.669999 66.700001) (end 112.370001 66.700001) (width 0.8) (layer "B.Cu") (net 4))
 (segment (start 112.370001 66.700001) (end 114.29 68.62) (width 0.8) (layer "B.Cu") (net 4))
 (segment (start 119.37 47.12) (end 119.37 47.38) (width 0.8) (layer "B.Cu") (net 4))
 (segment (start 103.049999 66.700001) (end 112.370001 66.700001) (width 0.8) (layer "B.Cu") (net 4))
 (segment (start 102.25 67.5) (end 103.049999 66.700001) (width 0.8) (layer "B.Cu") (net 4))
 (segment (start 116.75 58.54) (end 114.29 61) (width 0.8) (layer "B.Cu") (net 13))
 (segment (start 116.75 56) (end 116.75 58.54) (width 0.8) (layer "B.Cu") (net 13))
 (segment (start 111.5 56) (end 116.75 56) (width 0.8) (layer "B.Cu") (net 13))
 (segment (start 116.75 53.46) (end 116.75 56) (width 0.4) (layer "B.Cu") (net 13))
 (segment (start 109 56) (end 109 58.25) (width 0.8) (layer "B.Cu") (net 6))
 (segment (start 109 58.25) (end 111.75 61) (width 0.8) (layer "B.Cu") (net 6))
 (segment (start 109 47.75) (end 112 44.75) (width 0.8) (layer "B.Cu") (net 6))
 (segment (start 109 56) (end 109 47.75) (width 0.8) (layer "B.Cu") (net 6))
 (segment (start 100.96 59.75) (end 103.5 59.75) (width 0.8) (layer "B.Cu") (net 14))
 (segment (start 103.5 59.75) (end 107.96 59.75) (width 0.8) (layer "B.Cu") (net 14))
 (segment (start 107.96 59.75) (end 109.21 61) (width 0.8) (layer "B.Cu") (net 14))
 (segment (start 133.5 81.58) (end 134.645 81.58) (width 0.8) (layer "B.Cu") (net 8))
 (segment (start 139.475 76.75) (end 142.015 76.75) (width 0.8) (layer "B.Cu") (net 8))
 (segment (start 133.5 81.58) (end 124.45 72.53) (width 0.8) (layer "B.Cu") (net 8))
 (segment (start 134.645 81.58) (end 139.475 76.75) (width 0.8) (layer "B.Cu") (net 8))
 (segment (start 124.45 72.53) (end 124.45 68.62) (width 0.8) (layer "B.Cu") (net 8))
 (segment (start 122.015 75.25) (end 124.905844 75.25) (width 0.8) (layer "B.Cu") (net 2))
 (segment (start 143.666 77.433867) (end 143.666 75.166) (width 0.8) (layer "B.Cu") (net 2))
 (segment (start 143.666 70.876) (end 141.521 73.021) (width 0.8) (layer "B.Cu") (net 2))
 (segment (start 127.25 71.67) (end 127.25 63.8) (width 0.8) (layer "B.Cu") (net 2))
 (segment (start 143.666 75.166) (end 141.521 73.021) (width 0.8) (layer "B.Cu") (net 2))
 (segment (start 131.549867 42.2) (end 143.666 54.316133) (width 0.8) (layer "B.Cu") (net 2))
 (segment (start 119.475 75.25) (end 122.015 75.25) (width 0.8) (layer "B.Cu") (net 2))
 (segment (start 128.601 73.021) (end 127.25 71.67) (width 0.8) (layer "B.Cu") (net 2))
 (segment (start 143.666 54.316133) (end 143.666 70.876) (width 0.8) (layer "B.Cu") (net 2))
 (segment (start 132.836844 83.181) (end 137.918867 83.181) (width 0.8) (layer "B.Cu") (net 2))
 (segment (start 141.521 73.021) (end 128.601 73.021) (width 0.8) (layer "B.Cu") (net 2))
 (segment (start 137.918867 83.181) (end 143.666 77.433867) (width 0.8) (layer "B.Cu") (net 2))
 (segment (start 122 39.75) (end 124.45 42.2) (width 0.8) (layer "B.Cu") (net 2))
 (segment (start 124.45 42.2) (end 131.549867 42.2) (width 0.8) (layer "B.Cu") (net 2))
 (segment (start 124.905844 75.25) (end 132.836844 83.181) (width 0.8) (layer "B.Cu") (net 2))
 (segment (start 117 39.75) (end 122 39.75) (width 0.8) (layer "B.Cu") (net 2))
 (segment (start 127.25 63.8) (end 124.45 61) (width 0.8) (layer "B.Cu") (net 2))
 (segment (start 111.92 81.75) (end 116.83 76.84) (width 0.8) (layer "B.Cu") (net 5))
 (segment (start 116.83 76.84) (end 116.83 68.62) (width 0.8) (layer "B.Cu") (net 5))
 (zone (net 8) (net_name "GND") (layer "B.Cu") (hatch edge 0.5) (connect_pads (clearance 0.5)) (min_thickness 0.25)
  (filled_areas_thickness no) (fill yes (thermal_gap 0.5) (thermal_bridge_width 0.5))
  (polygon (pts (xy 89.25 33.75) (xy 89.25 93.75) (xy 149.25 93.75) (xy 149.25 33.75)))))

